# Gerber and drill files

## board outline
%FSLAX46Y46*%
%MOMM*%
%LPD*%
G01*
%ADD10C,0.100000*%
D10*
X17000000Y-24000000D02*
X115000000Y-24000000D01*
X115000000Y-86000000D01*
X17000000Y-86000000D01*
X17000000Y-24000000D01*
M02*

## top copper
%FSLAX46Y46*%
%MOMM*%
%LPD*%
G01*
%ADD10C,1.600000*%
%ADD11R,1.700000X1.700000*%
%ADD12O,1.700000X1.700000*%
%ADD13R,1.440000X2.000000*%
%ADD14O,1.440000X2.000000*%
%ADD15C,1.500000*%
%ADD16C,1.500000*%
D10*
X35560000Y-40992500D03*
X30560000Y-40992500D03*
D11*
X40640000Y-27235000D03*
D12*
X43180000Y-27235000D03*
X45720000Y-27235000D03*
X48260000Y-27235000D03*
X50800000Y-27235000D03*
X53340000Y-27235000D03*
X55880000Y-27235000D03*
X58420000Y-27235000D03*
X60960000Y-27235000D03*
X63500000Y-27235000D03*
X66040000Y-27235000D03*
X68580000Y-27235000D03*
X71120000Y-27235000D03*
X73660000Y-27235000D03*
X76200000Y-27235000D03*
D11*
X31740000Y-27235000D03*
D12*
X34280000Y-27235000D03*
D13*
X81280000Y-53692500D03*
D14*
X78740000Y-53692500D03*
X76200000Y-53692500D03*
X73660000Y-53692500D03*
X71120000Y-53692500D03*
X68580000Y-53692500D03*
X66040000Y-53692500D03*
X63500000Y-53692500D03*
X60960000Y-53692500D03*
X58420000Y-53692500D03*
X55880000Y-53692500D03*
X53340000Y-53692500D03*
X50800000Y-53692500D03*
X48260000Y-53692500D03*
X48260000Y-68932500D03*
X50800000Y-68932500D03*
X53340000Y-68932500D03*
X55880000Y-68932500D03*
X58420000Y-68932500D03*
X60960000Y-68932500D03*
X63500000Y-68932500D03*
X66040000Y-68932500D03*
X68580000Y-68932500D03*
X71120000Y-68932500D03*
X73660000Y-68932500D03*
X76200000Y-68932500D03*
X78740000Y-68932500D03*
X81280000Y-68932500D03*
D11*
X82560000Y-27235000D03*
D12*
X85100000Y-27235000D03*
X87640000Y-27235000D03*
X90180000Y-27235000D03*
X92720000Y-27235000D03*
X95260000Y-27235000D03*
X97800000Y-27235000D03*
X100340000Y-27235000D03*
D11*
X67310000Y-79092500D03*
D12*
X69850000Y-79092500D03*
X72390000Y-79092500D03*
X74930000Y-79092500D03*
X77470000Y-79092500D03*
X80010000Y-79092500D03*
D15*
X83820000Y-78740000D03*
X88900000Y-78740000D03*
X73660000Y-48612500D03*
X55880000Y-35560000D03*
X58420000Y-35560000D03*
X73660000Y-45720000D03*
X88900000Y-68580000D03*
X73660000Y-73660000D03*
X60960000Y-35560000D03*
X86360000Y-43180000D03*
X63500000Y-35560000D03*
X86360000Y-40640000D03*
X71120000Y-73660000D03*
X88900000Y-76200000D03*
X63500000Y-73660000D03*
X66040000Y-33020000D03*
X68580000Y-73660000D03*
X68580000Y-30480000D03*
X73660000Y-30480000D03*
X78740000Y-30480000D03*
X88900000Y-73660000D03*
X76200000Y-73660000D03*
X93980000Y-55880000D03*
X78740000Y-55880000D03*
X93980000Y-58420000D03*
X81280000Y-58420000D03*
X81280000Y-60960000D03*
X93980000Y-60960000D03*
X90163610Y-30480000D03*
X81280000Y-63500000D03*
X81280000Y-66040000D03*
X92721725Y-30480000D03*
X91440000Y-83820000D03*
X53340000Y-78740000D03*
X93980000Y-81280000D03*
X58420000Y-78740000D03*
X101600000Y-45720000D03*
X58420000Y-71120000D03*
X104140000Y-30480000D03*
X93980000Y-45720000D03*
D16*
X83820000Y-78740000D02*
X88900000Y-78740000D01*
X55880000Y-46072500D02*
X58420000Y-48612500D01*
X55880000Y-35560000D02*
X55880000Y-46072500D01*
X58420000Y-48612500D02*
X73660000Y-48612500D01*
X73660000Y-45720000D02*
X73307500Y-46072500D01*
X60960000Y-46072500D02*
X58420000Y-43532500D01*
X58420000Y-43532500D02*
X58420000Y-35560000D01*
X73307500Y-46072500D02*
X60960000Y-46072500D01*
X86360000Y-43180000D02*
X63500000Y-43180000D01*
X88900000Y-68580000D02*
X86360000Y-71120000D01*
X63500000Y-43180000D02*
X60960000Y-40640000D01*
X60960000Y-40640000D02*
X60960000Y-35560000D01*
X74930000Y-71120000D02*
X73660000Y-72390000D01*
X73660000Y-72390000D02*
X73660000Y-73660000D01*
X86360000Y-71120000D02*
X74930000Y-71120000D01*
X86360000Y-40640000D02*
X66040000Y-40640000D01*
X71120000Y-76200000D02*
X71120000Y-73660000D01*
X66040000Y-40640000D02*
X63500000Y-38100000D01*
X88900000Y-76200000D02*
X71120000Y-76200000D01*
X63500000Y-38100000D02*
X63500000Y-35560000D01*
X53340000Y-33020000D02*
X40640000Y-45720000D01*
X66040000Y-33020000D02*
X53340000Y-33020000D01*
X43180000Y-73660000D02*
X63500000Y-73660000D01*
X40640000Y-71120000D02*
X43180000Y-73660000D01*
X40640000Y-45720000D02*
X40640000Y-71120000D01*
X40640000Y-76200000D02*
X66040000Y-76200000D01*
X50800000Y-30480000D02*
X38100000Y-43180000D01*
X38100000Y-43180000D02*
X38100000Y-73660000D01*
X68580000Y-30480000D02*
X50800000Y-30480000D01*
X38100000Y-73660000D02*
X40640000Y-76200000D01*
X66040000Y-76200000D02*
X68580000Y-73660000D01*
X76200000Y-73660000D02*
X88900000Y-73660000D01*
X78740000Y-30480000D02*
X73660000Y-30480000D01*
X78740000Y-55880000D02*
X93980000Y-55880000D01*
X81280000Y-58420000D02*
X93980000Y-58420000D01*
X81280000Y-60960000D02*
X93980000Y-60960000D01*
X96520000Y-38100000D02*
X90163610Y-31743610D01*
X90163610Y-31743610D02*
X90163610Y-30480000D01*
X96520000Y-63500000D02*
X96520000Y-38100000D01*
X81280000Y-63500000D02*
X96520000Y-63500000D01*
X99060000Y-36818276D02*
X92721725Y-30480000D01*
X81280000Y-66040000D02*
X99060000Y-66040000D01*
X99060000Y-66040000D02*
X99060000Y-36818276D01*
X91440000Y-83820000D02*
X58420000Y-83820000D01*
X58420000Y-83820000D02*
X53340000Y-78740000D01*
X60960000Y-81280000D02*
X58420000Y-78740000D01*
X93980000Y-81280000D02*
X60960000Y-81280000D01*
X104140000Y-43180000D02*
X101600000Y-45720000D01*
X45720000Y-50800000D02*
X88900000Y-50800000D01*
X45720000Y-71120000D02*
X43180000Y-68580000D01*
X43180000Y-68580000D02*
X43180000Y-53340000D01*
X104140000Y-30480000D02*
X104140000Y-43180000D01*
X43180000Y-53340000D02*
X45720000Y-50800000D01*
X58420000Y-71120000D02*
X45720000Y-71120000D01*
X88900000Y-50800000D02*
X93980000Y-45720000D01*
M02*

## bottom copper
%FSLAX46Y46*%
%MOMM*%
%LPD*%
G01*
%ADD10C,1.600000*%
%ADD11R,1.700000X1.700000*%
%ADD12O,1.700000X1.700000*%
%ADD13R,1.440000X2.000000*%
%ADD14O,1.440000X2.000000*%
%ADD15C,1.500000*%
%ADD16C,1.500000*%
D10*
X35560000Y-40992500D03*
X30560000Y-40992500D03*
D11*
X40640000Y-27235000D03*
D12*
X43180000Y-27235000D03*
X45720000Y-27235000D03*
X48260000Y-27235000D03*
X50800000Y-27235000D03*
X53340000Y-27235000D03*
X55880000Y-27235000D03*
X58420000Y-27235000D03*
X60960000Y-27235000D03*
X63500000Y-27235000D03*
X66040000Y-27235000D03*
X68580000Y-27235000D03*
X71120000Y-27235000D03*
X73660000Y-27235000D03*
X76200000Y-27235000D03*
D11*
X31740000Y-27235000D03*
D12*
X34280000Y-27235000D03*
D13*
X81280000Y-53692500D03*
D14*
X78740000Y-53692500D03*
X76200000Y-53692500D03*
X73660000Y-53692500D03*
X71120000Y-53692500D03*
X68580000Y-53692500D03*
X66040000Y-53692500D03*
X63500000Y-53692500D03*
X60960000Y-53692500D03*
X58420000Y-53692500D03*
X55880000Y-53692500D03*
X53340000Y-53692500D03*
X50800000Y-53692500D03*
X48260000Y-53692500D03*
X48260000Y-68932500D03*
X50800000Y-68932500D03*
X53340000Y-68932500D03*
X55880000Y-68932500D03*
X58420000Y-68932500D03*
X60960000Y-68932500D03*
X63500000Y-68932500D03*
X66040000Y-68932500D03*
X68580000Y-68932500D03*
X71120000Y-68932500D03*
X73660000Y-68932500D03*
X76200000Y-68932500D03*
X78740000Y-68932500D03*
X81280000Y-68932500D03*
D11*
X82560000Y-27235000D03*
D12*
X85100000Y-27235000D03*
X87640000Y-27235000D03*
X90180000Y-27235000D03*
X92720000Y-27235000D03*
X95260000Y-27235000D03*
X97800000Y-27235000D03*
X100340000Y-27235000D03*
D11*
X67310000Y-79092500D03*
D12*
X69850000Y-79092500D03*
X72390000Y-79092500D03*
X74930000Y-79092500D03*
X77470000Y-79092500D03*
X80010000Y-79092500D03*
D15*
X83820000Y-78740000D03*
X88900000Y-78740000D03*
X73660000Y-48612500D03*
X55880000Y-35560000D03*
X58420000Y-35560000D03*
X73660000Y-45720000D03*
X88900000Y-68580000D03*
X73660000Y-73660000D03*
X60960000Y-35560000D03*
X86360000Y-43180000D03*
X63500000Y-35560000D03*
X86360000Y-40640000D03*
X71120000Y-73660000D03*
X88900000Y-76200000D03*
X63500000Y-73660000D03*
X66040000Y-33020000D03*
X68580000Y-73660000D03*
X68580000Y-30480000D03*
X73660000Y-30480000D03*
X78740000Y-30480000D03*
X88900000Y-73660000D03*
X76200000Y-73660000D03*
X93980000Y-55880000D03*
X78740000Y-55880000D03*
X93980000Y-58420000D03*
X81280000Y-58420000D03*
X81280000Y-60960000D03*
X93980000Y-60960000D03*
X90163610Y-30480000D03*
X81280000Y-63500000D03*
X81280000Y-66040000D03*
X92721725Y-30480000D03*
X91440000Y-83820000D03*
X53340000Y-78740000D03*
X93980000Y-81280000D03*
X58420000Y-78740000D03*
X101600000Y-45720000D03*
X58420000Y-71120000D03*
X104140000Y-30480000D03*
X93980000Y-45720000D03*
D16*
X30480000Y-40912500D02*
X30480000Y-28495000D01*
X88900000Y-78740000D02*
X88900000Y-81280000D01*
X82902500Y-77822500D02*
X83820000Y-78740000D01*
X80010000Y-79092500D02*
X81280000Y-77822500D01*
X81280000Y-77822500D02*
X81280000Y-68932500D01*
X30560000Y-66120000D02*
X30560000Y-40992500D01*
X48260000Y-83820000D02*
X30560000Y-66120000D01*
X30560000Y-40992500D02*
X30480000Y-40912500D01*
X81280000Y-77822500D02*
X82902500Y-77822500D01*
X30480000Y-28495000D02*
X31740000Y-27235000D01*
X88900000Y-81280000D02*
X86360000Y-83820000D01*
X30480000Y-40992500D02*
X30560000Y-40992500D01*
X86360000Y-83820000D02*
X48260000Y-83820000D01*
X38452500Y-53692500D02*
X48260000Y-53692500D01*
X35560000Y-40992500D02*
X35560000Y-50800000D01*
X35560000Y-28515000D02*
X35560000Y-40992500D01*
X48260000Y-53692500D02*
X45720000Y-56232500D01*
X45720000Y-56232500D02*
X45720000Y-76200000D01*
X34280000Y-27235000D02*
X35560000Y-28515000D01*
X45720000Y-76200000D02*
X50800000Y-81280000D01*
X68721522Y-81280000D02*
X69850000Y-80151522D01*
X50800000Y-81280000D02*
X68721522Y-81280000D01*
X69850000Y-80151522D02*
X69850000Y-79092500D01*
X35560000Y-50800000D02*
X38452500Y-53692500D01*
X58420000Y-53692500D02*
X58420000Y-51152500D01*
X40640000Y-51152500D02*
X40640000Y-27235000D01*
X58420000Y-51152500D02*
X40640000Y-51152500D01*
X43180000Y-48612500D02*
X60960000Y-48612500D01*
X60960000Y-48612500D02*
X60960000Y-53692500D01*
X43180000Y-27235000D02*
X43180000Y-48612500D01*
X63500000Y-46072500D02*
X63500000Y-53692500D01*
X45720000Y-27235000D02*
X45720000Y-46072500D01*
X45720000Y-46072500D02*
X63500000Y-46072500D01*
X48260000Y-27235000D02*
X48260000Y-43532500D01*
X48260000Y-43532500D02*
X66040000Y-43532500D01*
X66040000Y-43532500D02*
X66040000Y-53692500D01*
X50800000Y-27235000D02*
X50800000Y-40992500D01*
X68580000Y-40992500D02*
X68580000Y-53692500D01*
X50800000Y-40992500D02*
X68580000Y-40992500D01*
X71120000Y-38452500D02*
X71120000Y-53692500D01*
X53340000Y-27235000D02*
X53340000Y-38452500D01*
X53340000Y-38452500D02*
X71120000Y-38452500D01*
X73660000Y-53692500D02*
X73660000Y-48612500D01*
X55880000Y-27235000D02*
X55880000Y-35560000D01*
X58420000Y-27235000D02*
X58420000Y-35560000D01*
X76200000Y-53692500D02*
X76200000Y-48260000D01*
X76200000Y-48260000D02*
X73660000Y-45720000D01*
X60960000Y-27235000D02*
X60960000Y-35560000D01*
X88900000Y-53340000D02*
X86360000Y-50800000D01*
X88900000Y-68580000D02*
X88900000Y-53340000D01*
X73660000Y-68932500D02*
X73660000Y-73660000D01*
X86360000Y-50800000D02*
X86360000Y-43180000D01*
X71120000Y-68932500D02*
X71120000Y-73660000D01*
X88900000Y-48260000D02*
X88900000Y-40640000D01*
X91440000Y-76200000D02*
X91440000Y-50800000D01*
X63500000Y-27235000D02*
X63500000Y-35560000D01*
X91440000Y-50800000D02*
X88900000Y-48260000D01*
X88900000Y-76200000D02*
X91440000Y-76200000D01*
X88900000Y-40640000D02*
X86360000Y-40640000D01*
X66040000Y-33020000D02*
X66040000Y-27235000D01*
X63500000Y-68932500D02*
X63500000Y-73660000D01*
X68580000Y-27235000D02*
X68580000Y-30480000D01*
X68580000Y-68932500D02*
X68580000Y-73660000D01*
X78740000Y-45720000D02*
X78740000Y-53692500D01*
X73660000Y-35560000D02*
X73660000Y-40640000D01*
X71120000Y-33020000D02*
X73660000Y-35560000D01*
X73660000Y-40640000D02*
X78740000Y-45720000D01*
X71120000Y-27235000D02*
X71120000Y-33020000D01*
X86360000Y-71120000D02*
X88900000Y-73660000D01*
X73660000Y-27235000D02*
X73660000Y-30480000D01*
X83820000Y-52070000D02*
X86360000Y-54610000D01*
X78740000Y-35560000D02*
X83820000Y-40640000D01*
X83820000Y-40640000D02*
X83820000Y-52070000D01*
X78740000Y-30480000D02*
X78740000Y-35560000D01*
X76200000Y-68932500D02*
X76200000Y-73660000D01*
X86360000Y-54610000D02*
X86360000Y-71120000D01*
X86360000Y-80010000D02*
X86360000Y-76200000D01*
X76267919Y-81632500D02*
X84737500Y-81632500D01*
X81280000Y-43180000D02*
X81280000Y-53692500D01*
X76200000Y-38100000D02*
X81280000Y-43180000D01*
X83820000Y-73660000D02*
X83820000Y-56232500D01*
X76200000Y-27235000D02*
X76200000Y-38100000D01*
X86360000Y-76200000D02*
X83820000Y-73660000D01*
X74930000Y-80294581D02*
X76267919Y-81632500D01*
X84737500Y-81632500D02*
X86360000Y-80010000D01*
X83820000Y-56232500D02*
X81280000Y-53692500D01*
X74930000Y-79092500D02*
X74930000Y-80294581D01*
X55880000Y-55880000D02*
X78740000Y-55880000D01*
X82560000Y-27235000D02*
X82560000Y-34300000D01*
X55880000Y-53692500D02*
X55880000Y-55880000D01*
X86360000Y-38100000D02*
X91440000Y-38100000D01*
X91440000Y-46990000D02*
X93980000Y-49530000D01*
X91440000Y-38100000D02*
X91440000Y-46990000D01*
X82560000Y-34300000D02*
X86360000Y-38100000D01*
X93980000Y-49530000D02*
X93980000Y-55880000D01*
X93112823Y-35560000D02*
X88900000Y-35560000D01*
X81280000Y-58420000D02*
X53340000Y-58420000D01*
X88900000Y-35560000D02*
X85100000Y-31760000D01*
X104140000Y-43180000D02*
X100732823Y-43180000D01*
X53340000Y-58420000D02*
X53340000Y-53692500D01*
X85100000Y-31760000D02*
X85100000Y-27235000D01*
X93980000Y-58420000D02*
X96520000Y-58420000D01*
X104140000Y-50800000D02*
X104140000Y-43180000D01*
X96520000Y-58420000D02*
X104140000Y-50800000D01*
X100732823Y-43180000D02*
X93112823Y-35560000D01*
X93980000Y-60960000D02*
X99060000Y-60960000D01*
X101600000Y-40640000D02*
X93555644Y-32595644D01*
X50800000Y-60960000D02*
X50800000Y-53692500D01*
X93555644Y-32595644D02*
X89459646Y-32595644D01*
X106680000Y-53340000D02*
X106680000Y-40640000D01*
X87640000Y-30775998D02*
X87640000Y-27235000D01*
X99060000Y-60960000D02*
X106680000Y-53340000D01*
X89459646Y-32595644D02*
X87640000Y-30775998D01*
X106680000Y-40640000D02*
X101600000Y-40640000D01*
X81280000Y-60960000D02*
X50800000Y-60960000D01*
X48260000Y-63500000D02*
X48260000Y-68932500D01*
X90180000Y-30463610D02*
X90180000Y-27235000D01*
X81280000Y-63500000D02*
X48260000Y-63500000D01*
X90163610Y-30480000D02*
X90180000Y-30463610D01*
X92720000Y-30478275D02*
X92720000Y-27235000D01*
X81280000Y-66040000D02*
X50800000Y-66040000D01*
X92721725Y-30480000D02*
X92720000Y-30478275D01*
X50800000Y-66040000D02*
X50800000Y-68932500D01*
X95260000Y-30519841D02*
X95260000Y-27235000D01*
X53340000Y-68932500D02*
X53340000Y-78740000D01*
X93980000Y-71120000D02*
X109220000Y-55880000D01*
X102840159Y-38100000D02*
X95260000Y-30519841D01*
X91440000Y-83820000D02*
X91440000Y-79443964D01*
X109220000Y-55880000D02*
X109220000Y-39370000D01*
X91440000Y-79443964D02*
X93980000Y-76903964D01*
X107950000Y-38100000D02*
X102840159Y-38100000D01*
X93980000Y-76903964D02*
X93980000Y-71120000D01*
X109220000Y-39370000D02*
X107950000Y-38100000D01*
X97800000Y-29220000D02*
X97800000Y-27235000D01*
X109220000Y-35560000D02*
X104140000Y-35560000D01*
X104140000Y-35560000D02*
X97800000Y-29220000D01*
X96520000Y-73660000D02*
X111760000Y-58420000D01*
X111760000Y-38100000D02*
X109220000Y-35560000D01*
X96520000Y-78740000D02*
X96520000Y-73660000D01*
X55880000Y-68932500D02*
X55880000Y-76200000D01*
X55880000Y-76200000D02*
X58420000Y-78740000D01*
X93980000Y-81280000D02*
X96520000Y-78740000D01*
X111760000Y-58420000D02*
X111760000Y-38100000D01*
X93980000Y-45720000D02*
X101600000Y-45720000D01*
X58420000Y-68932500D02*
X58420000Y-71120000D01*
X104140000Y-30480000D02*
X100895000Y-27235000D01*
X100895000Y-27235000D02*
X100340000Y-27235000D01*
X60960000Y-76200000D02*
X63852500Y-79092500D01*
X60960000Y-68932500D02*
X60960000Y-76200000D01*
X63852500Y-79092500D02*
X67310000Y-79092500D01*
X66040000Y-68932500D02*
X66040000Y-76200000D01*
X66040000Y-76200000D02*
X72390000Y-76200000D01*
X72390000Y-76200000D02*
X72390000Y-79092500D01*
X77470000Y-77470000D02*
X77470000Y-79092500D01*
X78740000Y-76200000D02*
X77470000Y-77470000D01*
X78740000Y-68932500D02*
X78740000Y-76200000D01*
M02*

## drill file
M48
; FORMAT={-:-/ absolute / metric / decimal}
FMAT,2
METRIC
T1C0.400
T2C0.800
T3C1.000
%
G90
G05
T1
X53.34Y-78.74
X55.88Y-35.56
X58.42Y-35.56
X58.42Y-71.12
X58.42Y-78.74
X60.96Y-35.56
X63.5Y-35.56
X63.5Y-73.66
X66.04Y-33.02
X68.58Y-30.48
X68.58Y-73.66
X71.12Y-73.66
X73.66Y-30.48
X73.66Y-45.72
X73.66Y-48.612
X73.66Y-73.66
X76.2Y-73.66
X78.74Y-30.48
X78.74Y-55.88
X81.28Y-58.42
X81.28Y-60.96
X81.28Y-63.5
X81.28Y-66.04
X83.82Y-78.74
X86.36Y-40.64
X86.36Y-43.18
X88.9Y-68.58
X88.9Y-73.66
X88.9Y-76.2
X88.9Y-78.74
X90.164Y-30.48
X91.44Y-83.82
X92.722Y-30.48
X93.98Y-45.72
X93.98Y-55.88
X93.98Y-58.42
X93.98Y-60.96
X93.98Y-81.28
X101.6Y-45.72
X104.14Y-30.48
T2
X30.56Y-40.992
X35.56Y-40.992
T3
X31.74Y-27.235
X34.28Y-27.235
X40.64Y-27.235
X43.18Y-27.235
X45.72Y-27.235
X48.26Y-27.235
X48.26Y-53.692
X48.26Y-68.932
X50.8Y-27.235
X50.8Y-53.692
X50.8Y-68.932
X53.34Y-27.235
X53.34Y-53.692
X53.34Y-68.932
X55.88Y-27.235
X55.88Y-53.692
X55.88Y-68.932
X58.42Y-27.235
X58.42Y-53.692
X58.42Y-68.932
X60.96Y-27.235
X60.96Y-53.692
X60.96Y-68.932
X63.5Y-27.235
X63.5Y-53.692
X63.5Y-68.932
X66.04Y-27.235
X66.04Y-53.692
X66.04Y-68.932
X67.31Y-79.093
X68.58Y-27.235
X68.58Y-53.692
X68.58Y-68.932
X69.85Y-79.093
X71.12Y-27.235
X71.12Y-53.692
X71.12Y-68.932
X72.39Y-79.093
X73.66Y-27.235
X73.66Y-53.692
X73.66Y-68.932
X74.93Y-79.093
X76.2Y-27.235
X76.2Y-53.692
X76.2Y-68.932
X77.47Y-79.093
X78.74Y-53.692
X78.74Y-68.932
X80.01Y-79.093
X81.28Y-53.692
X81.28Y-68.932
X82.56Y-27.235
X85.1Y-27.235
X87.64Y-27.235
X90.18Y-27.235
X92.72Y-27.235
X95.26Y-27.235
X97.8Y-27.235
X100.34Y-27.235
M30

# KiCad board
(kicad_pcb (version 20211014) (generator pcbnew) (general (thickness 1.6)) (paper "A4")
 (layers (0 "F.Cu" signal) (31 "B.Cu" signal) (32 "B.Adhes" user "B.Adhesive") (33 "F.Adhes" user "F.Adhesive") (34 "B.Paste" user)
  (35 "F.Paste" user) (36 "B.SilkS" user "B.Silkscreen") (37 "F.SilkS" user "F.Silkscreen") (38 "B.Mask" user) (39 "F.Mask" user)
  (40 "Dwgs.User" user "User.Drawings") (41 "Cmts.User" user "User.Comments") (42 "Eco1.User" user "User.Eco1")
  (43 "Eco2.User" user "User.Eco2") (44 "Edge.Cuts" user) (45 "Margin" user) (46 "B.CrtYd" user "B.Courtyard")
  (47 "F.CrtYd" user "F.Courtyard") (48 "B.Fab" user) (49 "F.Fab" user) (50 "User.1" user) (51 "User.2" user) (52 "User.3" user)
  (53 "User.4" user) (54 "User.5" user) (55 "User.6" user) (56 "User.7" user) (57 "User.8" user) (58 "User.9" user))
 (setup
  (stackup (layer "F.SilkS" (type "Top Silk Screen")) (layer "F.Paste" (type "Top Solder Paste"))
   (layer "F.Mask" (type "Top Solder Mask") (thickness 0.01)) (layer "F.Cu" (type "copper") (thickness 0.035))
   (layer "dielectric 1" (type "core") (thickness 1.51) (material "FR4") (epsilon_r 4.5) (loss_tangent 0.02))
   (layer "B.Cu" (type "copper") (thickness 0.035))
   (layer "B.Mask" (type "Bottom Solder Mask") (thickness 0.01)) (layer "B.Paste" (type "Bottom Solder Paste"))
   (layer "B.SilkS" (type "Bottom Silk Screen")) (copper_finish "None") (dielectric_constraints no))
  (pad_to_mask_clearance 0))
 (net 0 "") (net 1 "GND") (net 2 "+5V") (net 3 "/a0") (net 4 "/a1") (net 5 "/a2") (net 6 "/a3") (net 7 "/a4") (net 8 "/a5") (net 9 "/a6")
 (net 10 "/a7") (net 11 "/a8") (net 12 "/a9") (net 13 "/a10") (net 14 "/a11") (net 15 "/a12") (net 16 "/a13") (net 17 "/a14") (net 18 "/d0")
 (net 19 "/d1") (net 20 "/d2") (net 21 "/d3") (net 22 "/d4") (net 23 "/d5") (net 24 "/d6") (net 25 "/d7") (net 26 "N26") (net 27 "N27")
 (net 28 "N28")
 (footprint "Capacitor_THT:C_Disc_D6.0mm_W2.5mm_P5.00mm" (layer "F.Cu") (at 35.56 40.9925 180)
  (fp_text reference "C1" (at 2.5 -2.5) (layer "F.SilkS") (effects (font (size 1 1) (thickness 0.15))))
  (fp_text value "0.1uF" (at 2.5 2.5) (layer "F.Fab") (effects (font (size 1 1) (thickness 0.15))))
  (pad "1" thru_hole circle locked (at 0 0 180) (size 1.6 1.6) (drill 0.8) (layers *.Cu *.Mask) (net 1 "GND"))
  (pad "2" thru_hole circle locked (at 5 0 180) (size 1.6 1.6) (drill 0.8) (layers *.Cu *.Mask) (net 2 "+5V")))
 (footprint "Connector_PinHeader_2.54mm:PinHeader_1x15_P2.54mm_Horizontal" (layer "F.Cu") (at 40.64 27.235 90)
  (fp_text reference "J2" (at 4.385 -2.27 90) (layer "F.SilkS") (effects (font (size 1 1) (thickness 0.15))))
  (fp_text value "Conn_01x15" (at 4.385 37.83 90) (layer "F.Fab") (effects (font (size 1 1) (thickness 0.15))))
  (pad "1" thru_hole rect locked (at 0 0 90) (size 1.7 1.7) (drill 1) (layers *.Cu *.Mask) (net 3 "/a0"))
  (pad "2" thru_hole oval locked (at 0 2.54 90) (size 1.7 1.7) (drill 1) (layers *.Cu *.Mask) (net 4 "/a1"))
  (pad "3" thru_hole oval locked (at 0 5.08 90) (size 1.7 1.7) (drill 1) (layers *.Cu *.Mask) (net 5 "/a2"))
  (pad "4" thru_hole oval locked (at 0 7.62 90) (size 1.7 1.7) (drill 1) (layers *.Cu *.Mask) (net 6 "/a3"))
  (pad "5" thru_hole oval locked (at 0 10.16 90) (size 1.7 1.7) (drill 1) (layers *.Cu *.Mask) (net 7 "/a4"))
  (pad "6" thru_hole oval locked (at 0 12.7 90) (size 1.7 1.7) (drill 1) (layers *.Cu *.Mask) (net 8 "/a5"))
  (pad "7" thru_hole oval locked (at 0 15.24 90) (size 1.7 1.7) (drill 1) (layers *.Cu *.Mask) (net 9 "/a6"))
  (pad "8" thru_hole oval locked (at 0 17.78 90) (size 1.7 1.7) (drill 1) (layers *.Cu *.Mask) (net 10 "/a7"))
  (pad "9" thru_hole oval locked (at 0 20.32 90) (size 1.7 1.7) (drill 1) (layers *.Cu *.Mask) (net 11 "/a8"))
  (pad "10" thru_hole oval locked (at 0 22.86 90) (size 1.7 1.7) (drill 1) (layers *.Cu *.Mask) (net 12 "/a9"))
  (pad "11" thru_hole oval locked (at 0 25.4 90) (size 1.7 1.7) (drill 1) (layers *.Cu *.Mask) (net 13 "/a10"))
  (pad "12" thru_hole oval locked (at 0 27.94 90) (size 1.7 1.7) (drill 1) (layers *.Cu *.Mask) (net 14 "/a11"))
  (pad "13" thru_hole oval locked (at 0 30.48 90) (size 1.7 1.7) (drill 1) (layers *.Cu *.Mask) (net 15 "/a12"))
  (pad "14" thru_hole oval locked (at 0 33.02 90) (size 1.7 1.7) (drill 1) (layers *.Cu *.Mask) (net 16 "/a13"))
  (pad "15" thru_hole oval locked (at 0 35.56 90) (size 1.7 1.7) (drill 1) (layers *.Cu *.Mask) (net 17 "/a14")))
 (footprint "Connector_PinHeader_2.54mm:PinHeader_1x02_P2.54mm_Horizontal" (layer "F.Cu") (at 31.74 27.235 90)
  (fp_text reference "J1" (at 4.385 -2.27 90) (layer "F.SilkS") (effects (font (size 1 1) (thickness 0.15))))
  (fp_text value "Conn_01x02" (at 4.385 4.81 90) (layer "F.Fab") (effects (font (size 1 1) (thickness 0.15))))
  (pad "1" thru_hole rect locked (at 0 0 90) (size 1.7 1.7) (drill 1) (layers *.Cu *.Mask) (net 2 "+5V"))
  (pad "2" thru_hole oval locked (at 0 2.54 90) (size 1.7 1.7) (drill 1) (layers *.Cu *.Mask) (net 1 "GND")))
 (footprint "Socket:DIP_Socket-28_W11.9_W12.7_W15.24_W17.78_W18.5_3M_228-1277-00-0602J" (layer "F.Cu") (at 81.28 53.6925 -90)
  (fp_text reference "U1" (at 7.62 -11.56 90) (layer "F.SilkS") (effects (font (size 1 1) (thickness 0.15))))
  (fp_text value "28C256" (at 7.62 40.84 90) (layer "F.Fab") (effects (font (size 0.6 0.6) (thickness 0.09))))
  (pad "1" thru_hole rect locked (at 0 0 270) (size 2 1.44) (drill 1) (layers *.Cu *.Mask) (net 17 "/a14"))
  (pad "2" thru_hole oval locked (at 0 2.54 270) (size 2 1.44) (drill 1) (layers *.Cu *.Mask) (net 15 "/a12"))
  (pad "3" thru_hole oval locked (at 0 5.08 270) (size 2 1.44) (drill 1) (layers *.Cu *.Mask) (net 10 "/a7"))
  (pad "4" thru_hole oval locked (at 0 7.62 270) (size 2 1.44) (drill 1) (layers *.Cu *.Mask) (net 9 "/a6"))
  (pad "5" thru_hole oval locked (at 0 10.16 270) (size 2 1.44) (drill 1) (layers *.Cu *.Mask) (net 8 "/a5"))
  (pad "6" thru_hole oval locked (at 0 12.7 270) (size 2 1.44) (drill 1) (layers *.Cu *.Mask) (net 7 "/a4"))
  (pad "7" thru_hole oval locked (at 0 15.24 270) (size 2 1.44) (drill 1) (layers *.Cu *.Mask) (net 6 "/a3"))
  (pad "8" thru_hole oval locked (at 0 17.78 270) (size 2 1.44) (drill 1) (layers *.Cu *.Mask) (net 5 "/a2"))
  (pad "9" thru_hole oval locked (at 0 20.32 270) (size 2 1.44) (drill 1) (layers *.Cu *.Mask) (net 4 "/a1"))
  (pad "10" thru_hole oval locked (at 0 22.86 270) (size 2 1.44) (drill 1) (layers *.Cu *.Mask) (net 3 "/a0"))
  (pad "11" thru_hole oval locked (at 0 25.4 270) (size 2 1.44) (drill 1) (layers *.Cu *.Mask) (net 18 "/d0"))
  (pad "12" thru_hole oval locked (at 0 27.94 270) (size 2 1.44) (drill 1) (layers *.Cu *.Mask) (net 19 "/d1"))
  (pad "13" thru_hole oval locked (at 0 30.48 270) (size 2 1.44) (drill 1) (layers *.Cu *.Mask) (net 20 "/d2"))
  (pad "14" thru_hole oval locked (at 0 33.02 270) (size 2 1.44) (drill 1) (layers *.Cu *.Mask) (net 1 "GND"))
  (pad "15" thru_hole oval locked (at 15.24 33.02 270) (size 2 1.44) (drill 1) (layers *.Cu *.Mask) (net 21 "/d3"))
  (pad "16" thru_hole oval locked (at 15.24 30.48 270) (size 2 1.44) (drill 1) (layers *.Cu *.Mask) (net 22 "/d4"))
  (pad "17" thru_hole oval locked (at 15.24 27.94 270) (size 2 1.44) (drill 1) (layers *.Cu *.Mask) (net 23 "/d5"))
  (pad "18" thru_hole oval locked (at 15.24 25.4 270) (size 2 1.44) (drill 1) (layers *.Cu *.Mask) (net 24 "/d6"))
  (pad "19" thru_hole oval locked (at 15.24 22.86 270) (size 2 1.44) (drill 1) (layers *.Cu *.Mask) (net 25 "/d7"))
  (pad "20" thru_hole oval locked (at 15.24 20.32 270) (size 2 1.44) (drill 1) (layers *.Cu *.Mask) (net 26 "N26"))
  (pad "21" thru_hole oval locked (at 15.24 17.78 270) (size 2 1.44) (drill 1) (layers *.Cu *.Mask) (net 13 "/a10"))
  (pad "22" thru_hole oval locked (at 15.24 15.24 270) (size 2 1.44) (drill 1) (layers *.Cu *.Mask) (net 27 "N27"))
  (pad "23" thru_hole oval locked (at 15.24 12.7 270) (size 2 1.44) (drill 1) (layers *.Cu *.Mask) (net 14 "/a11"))
  (pad "24" thru_hole oval locked (at 15.24 10.16 270) (size 2 1.44) (drill 1) (layers *.Cu *.Mask) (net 12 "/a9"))
  (pad "25" thru_hole oval locked (at 15.24 7.62 270) (size 2 1.44) (drill 1) (layers *.Cu *.Mask) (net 11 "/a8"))
  (pad "26" thru_hole oval locked (at 15.24 5.08 270) (size 2 1.44) (drill 1) (layers *.Cu *.Mask) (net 16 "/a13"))
  (pad "27" thru_hole oval locked (at 15.24 2.54 270) (size 2 1.44) (drill 1) (layers *.Cu *.Mask) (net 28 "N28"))
  (pad "28" thru_hole oval locked (at 15.24 0 270) (size 2 1.44) (drill 1) (layers *.Cu *.Mask) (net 2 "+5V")))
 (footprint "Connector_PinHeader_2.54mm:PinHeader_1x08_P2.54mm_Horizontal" (layer "F.Cu") (at 82.56 27.235 90)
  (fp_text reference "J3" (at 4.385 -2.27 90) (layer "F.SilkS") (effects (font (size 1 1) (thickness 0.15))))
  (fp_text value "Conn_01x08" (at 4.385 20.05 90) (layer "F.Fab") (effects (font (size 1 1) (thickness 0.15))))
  (pad "1" thru_hole rect locked (at 0 0 90) (size 1.7 1.7) (drill 1) (layers *.Cu *.Mask) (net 18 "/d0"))
  (pad "2" thru_hole oval locked (at 0 2.54 90) (size 1.7 1.7) (drill 1) (layers *.Cu *.Mask) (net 19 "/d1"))
  (pad "3" thru_hole oval locked (at 0 5.08 90) (size 1.7 1.7) (drill 1) (layers *.Cu *.Mask) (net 20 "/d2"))
  (pad "4" thru_hole oval locked (at 0 7.62 90) (size 1.7 1.7) (drill 1) (layers *.Cu *.Mask) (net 21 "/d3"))
  (pad "5" thru_hole oval locked (at 0 10.16 90) (size 1.7 1.7) (drill 1) (layers *.Cu *.Mask) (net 22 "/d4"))
  (pad "6" thru_hole oval locked (at 0 12.7 90) (size 1.7 1.7) (drill 1) (layers *.Cu *.Mask) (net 23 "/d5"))
  (pad "7" thru_hole oval locked (at 0 15.24 90) (size 1.7 1.7) (drill 1) (layers *.Cu *.Mask) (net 24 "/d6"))
  (pad "8" thru_hole oval locked (at 0 17.78 90) (size 1.7 1.7) (drill 1) (layers *.Cu *.Mask) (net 25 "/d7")))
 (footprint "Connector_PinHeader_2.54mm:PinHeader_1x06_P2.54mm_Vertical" (layer "F.Cu") (at 67.31 79.0925 90)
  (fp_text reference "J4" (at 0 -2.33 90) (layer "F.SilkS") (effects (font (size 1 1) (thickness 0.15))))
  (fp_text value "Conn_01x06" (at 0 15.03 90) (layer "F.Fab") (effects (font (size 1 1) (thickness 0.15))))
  (pad "1" thru_hole rect locked (at 0 0 90) (size 1.7 1.7) (drill 1) (layers *.Cu *.Mask) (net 26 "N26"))
  (pad "2" thru_hole oval locked (at 0 2.54 90) (size 1.7 1.7) (drill 1) (layers *.Cu *.Mask) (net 1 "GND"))
  (pad "3" thru_hole oval locked (at 0 5.08 90) (size 1.7 1.7) (drill 1) (layers *.Cu *.Mask) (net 27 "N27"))
  (pad "4" thru_hole oval locked (at 0 7.62 90) (size 1.7 1.7) (drill 1) (layers *.Cu *.Mask) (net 17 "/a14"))
  (pad "5" thru_hole oval locked (at 0 10.16 90) (size 1.7 1.7) (drill 1) (layers *.Cu *.Mask) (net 28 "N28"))
  (pad "6" thru_hole oval locked (at 0 12.7 90) (size 1.7 1.7) (drill 1) (layers *.Cu *.Mask) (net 2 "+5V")))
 (gr_rect (start 17 24) (end 115 86) (layer "Edge.Cuts") (width 0.1) (fill none))
 (segment (start 83.82 78.74) (end 88.9 78.74) (width 1.5) (layer "F.Cu") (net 2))
 (via (at 83.82 78.74) (size 1.5) (drill 0.4) (layers "F.Cu" "B.Cu") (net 2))
 (via (at 88.9 78.74) (size 1.5) (drill 0.4) (layers "F.Cu" "B.Cu") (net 2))
 (segment (start 30.48 40.9125) (end 30.48 28.495) (width 1.5) (layer "B.Cu") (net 2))
 (segment (start 88.9 78.74) (end 88.9 81.28) (width 1.5) (layer "B.Cu") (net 2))
 (segment (start 82.9025 77.8225) (end 83.82 78.74) (width 1.5) (layer "B.Cu") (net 2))
 (segment (start 80.01 79.0925) (end 81.28 77.8225) (width 1.5) (layer "B.Cu") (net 2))
 (segment (start 81.28 77.8225) (end 81.28 68.9325) (width 1.5) (layer "B.Cu") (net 2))
 (segment (start 30.56 66.12) (end 30.56 40.9925) (width 1.5) (layer "B.Cu") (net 2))
 (segment (start 48.26 83.82) (end 30.56 66.12) (width 1.5) (layer "B.Cu") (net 2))
 (segment (start 30.56 40.9925) (end 30.48 40.9125) (width 1.5) (layer "B.Cu") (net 2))
 (segment (start 81.28 77.8225) (end 82.9025 77.8225) (width 1.5) (layer "B.Cu") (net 2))
 (segment (start 30.48 28.495) (end 31.74 27.235) (width 1.5) (layer "B.Cu") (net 2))
 (segment (start 88.9 81.28) (end 86.36 83.82) (width 1.5) (layer "B.Cu") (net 2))
 (segment (start 30.48 40.9925) (end 30.56 40.9925) (width 1.5) (layer "B.Cu") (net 2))
 (segment (start 86.36 83.82) (end 48.26 83.82) (width 1.5) (layer "B.Cu") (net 2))
 (segment (start 38.4525 53.6925) (end 48.26 53.6925) (width 1.5) (layer "B.Cu") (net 1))
 (segment (start 35.56 40.9925) (end 35.56 50.8) (width 1.5) (layer "B.Cu") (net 1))
 (segment (start 35.56 28.515) (end 35.56 40.9925) (width 1.5) (layer "B.Cu") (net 1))
 (segment (start 48.26 53.6925) (end 45.72 56.2325) (width 1.5) (layer "B.Cu") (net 1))
 (segment (start 45.72 56.2325) (end 45.72 76.2) (width 1.5) (layer "B.Cu") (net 1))
 (segment (start 34.28 27.235) (end 35.56 28.515) (width 1.5) (layer "B.Cu") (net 1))
 (segment (start 45.72 76.2) (end 50.8 81.28) (width 1.5) (layer "B.Cu") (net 1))
 (segment (start 68.721522 81.28) (end 69.85 80.151522) (width 1.5) (layer "B.Cu") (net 1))
 (segment (start 50.8 81.28) (end 68.721522 81.28) (width 1.5) (layer "B.Cu") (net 1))
 (segment (start 69.85 80.151522) (end 69.85 79.0925) (width 1.5) (layer "B.Cu") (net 1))
 (segment (start 35.56 50.8) (end 38.4525 53.6925) (width 1.5) (layer "B.Cu") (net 1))
 (segment (start 58.42 53.6925) (end 58.42 51.1525) (width 1.5) (layer "B.Cu") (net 3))
 (segment (start 40.64 51.1525) (end 40.64 27.235) (width 1.5) (layer "B.Cu") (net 3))
 (segment (start 58.42 51.1525) (end 40.64 51.1525) (width 1.5) (layer "B.Cu") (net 3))
 (segment (start 43.18 48.6125) (end 60.96 48.6125) (width 1.5) (layer "B.Cu") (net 4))
 (segment (start 60.96 48.6125) (end 60.96 53.6925) (width 1.5) (layer "B.Cu") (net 4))
 (segment (start 43.18 27.235) (end 43.18 48.6125) (width 1.5) (layer "B.Cu") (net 4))
 (segment (start 63.5 46.0725) (end 63.5 53.6925) (width 1.5) (layer "B.Cu") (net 5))
 (segment (start 45.72 27.235) (end 45.72 46.0725) (width 1.5) (layer "B.Cu") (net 5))
 (segment (start 45.72 46.0725) (end 63.5 46.0725) (width 1.5) (layer "B.Cu") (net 5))
 (segment (start 48.26 27.235) (end 48.26 43.5325) (width 1.5) (layer "B.Cu") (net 6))
 (segment (start 48.26 43.5325) (end 66.04 43.5325) (width 1.5) (layer "B.Cu") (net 6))
 (segment (start 66.04 43.5325) (end 66.04 53.6925) (width 1.5) (layer "B.Cu") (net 6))
 (segment (start 50.8 27.235) (end 50.8 40.9925) (width 1.5) (layer "B.Cu") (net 7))
 (segment (start 68.58 40.9925) (end 68.58 53.6925) (width 1.5) (layer "B.Cu") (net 7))
 (segment (start 50.8 40.9925) (end 68.58 40.9925) (width 1.5) (layer "B.Cu") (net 7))
 (segment (start 71.12 38.4525) (end 71.12 53.6925) (width 1.5) (layer "B.Cu") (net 8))
 (segment (start 53.34 27.235) (end 53.34 38.4525) (width 1.5) (layer "B.Cu") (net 8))
 (segment (start 53.34 38.4525) (end 71.12 38.4525) (width 1.5) (layer "B.Cu") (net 8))
 (segment (start 55.88 46.0725) (end 58.42 48.6125) (width 1.5) (layer "F.Cu") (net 9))
 (segment (start 55.88 35.56) (end 55.88 46.0725) (width 1.5) (layer "F.Cu") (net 9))
 (segment (start 58.42 48.6125) (end 73.66 48.6125) (width 1.5) (layer "F.Cu") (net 9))
 (via (at 73.66 48.6125) (size 1.5) (drill 0.4) (layers "F.Cu" "B.Cu") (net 9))
 (via (at 55.88 35.56) (size 1.5) (drill 0.4) (layers "F.Cu" "B.Cu") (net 9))
 (segment (start 73.66 53.6925) (end 73.66 48.6125) (width 1.5) (layer "B.Cu") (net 9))
 (segment (start 55.88 27.235) (end 55.88 35.56) (width 1.5) (layer "B.Cu") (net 9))
 (segment (start 73.66 45.72) (end 73.3075 46.0725) (width 1.5) (layer "F.Cu") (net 10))
 (segment (start 60.96 46.0725) (end 58.42 43.5325) (width 1.5) (layer "F.Cu") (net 10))
 (segment (start 58.42 43.5325) (end 58.42 35.56) (width 1.5) (layer "F.Cu") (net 10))
 (segment (start 73.3075 46.0725) (end 60.96 46.0725) (width 1.5) (layer "F.Cu") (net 10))
 (via (at 58.42 35.56) (size 1.5) (drill 0.4) (layers "F.Cu" "B.Cu") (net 10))
 (via (at 73.66 45.72) (size 1.5) (drill 0.4) (layers "F.Cu" "B.Cu") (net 10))
 (segment (start 58.42 27.235) (end 58.42 35.56) (width 1.5) (layer "B.Cu") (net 10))
 (segment (start 76.2 53.6925) (end 76.2 48.26) (width 1.5) (layer "B.Cu") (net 10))
 (segment (start 76.2 48.26) (end 73.66 45.72) (width 1.5) (layer "B.Cu") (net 10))
 (segment (start 86.36 43.18) (end 63.5 43.18) (width 1.5) (layer "F.Cu") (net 11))
 (segment (start 88.9 68.58) (end 86.36 71.12) (width 1.5) (layer "F.Cu") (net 11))
 (segment (start 63.5 43.18) (end 60.96 40.64) (width 1.5) (layer "F.Cu") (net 11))
 (segment (start 60.96 40.64) (end 60.96 35.56) (width 1.5) (layer "F.Cu") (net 11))
 (segment (start 74.93 71.12) (end 73.66 72.39) (width 1.5) (layer "F.Cu") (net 11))
 (segment (start 73.66 72.39) (end 73.66 73.66) (width 1.5) (layer "F.Cu") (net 11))
 (segment (start 86.36 71.12) (end 74.93 71.12) (width 1.5) (layer "F.Cu") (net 11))
 (via (at 88.9 68.58) (size 1.5) (drill 0.4) (layers "F.Cu" "B.Cu") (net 11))
 (via (at 73.66 73.66) (size 1.5) (drill 0.4) (layers "F.Cu" "B.Cu") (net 11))
 (via (at 60.96 35.56) (size 1.5) (drill 0.4) (layers "F.Cu" "B.Cu") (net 11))
 (via (at 86.36 43.18) (size 1.5) (drill 0.4) (layers "F.Cu" "B.Cu") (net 11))
 (segment (start 60.96 27.235) (end 60.96 35.56) (width 1.5) (layer "B.Cu") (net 11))
 (segment (start 88.9 53.34) (end 86.36 50.8) (width 1.5) (layer "B.Cu") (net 11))
 (segment (start 88.9 68.58) (end 88.9 53.34) (width 1.5) (layer "B.Cu") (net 11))
 (segment (start 73.66 68.9325) (end 73.66 73.66) (width 1.5) (layer "B.Cu") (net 11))
 (segment (start 86.36 50.8) (end 86.36 43.18) (width 1.5) (layer "B.Cu") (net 11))
 (segment (start 86.36 40.64) (end 66.04 40.64) (width 1.5) (layer "F.Cu") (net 12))
 (segment (start 71.12 76.2) (end 71.12 73.66) (width 1.5) (layer "F.Cu") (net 12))
 (segment (start 66.04 40.64) (end 63.5 38.1) (width 1.5) (layer "F.Cu") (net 12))
 (segment (start 88.9 76.2) (end 71.12 76.2) (width 1.5) (layer "F.Cu") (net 12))
 (segment (start 63.5 38.1) (end 63.5 35.56) (width 1.5) (layer "F.Cu") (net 12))
 (via (at 63.5 35.56) (size 1.5) (drill 0.4) (layers "F.Cu" "B.Cu") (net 12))
 (via (at 86.36 40.64) (size 1.5) (drill 0.4) (layers "F.Cu" "B.Cu") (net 12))
 (via (at 71.12 73.66) (size 1.5) (drill 0.4) (layers "F.Cu" "B.Cu") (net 12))
 (via (at 88.9 76.2) (size 1.5) (drill 0.4) (layers "F.Cu" "B.Cu") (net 12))
 (segment (start 71.12 68.9325) (end 71.12 73.66) (width 1.5) (layer "B.Cu") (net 12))
 (segment (start 88.9 48.26) (end 88.9 40.64) (width 1.5) (layer "B.Cu") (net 12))
 (segment (start 91.44 76.2) (end 91.44 50.8) (width 1.5) (layer "B.Cu") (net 12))
 (segment (start 63.5 27.235) (end 63.5 35.56) (width 1.5) (layer "B.Cu") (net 12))
 (segment (start 91.44 50.8) (end 88.9 48.26) (width 1.5) (layer "B.Cu") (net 12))
 (segment (start 88.9 76.2) (end 91.44 76.2) (width 1.5) (layer "B.Cu") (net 12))
 (segment (start 88.9 40.64) (end 86.36 40.64) (width 1.5) (layer "B.Cu") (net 12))
 (segment (start 53.34 33.02) (end 40.64 45.72) (width 1.5) (layer "F.Cu") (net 13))
 (segment (start 66.04 33.02) (end 53.34 33.02) (width 1.5) (layer "F.Cu") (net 13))
 (segment (start 43.18 73.66) (end 63.5 73.66) (width 1.5) (layer "F.Cu") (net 13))
 (segment (start 40.64 71.12) (end 43.18 73.66) (width 1.5) (layer "F.Cu") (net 13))
 (segment (start 40.64 45.72) (end 40.64 71.12) (width 1.5) (layer "F.Cu") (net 13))
 (via (at 63.5 73.66) (size 1.5) (drill 0.4) (layers "F.Cu" "B.Cu") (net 13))
 (via (at 66.04 33.02) (size 1.5) (drill 0.4) (layers "F.Cu" "B.Cu") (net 13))
 (segment (start 66.04 33.02) (end 66.04 27.235) (width 1.5) (layer "B.Cu") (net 13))
 (segment (start 63.5 68.9325) (end 63.5 73.66) (width 1.5) (layer "B.Cu") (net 13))
 (segment (start 40.64 76.2) (end 66.04 76.2) (width 1.5) (layer "F.Cu") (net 14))
 (segment (start 50.8 30.48) (end 38.1 43.18) (width 1.5) (layer "F.Cu") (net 14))
 (segment (start 38.1 43.18) (end 38.1 73.66) (width 1.5) (layer "F.Cu") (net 14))
 (segment (start 68.58 30.48) (end 50.8 30.48) (width 1.5) (layer "F.Cu") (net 14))
 (segment (start 38.1 73.66) (end 40.64 76.2) (width 1.5) (layer "F.Cu") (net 14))
 (segment (start 66.04 76.2) (end 68.58 73.66) (width 1.5) (layer "F.Cu") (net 14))
 (via (at 68.58 73.66) (size 1.5) (drill 0.4) (layers "F.Cu" "B.Cu") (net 14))
 (via (at 68.58 30.48) (size 1.5) (drill 0.4) (layers "F.Cu" "B.Cu") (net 14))
 (segment (start 68.58 27.235) (end 68.58 30.48) (width 1.5) (layer "B.Cu") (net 14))
 (segment (start 68.58 68.9325) (end 68.58 73.66) (width 1.5) (layer "B.Cu") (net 14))
 (segment (start 78.74 45.72) (end 78.74 53.6925) (width 1.5) (layer "B.Cu") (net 15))
 (segment (start 73.66 35.56) (end 73.66 40.64) (width 1.5) (layer "B.Cu") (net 15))
 (segment (start 71.12 33.02) (end 73.66 35.56) (width 1.5) (layer "B.Cu") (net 15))
 (segment (start 73.66 40.64) (end 78.74 45.72) (width 1.5) (layer "B.Cu") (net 15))
 (segment (start 71.12 27.235) (end 71.12 33.02) (width 1.5) (layer "B.Cu") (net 15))
 (segment (start 76.2 73.66) (end 88.9 73.66) (width 1.5) (layer "F.Cu") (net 16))
 (segment (start 78.74 30.48) (end 73.66 30.48) (width 1.5) (layer "F.Cu") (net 16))
 (via (at 73.66 30.48) (size 1.5) (drill 0.4) (layers "F.Cu" "B.Cu") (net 16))
 (via (at 78.74 30.48) (size 1.5) (drill 0.4) (layers "F.Cu" "B.Cu") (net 16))
 (via (at 88.9 73.66) (size 1.5) (drill 0.4) (layers "F.Cu" "B.Cu") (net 16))
 (via (at 76.2 73.66) (size 1.5) (drill 0.4) (layers "F.Cu" "B.Cu") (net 16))
 (segment (start 86.36 71.12) (end 88.9 73.66) (width 1.5) (layer "B.Cu") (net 16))
 (segment (start 73.66 27.235) (end 73.66 30.48) (width 1.5) (layer "B.Cu") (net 16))
 (segment (start 83.82 52.07) (end 86.36 54.61) (width 1.5) (layer "B.Cu") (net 16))
 (segment (start 78.74 35.56) (end 83.82 40.64) (width 1.5) (layer "B.Cu") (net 16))
 (segment (start 83.82 40.64) (end 83.82 52.07) (width 1.5) (layer "B.Cu") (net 16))
 (segment (start 78.74 30.48) (end 78.74 35.56) (width 1.5) (layer "B.Cu") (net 16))
 (segment (start 76.2 68.9325) (end 76.2 73.66) (width 1.5) (layer "B.Cu") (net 16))
 (segment (start 86.36 54.61) (end 86.36 71.12) (width 1.5) (layer "B.Cu") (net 16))
 (segment (start 86.36 80.01) (end 86.36 76.2) (width 1.5) (layer "B.Cu") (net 17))
 (segment (start 76.267919 81.6325) (end 84.7375 81.6325) (width 1.5) (layer "B.Cu") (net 17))
 (segment (start 81.28 43.18) (end 81.28 53.6925) (width 1.5) (layer "B.Cu") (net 17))
 (segment (start 76.2 38.1) (end 81.28 43.18) (width 1.5) (layer "B.Cu") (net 17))
 (segment (start 83.82 73.66) (end 83.82 56.2325) (width 1.5) (layer "B.Cu") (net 17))
 (segment (start 76.2 27.235) (end 76.2 38.1) (width 1.5) (layer "B.Cu") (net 17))
 (segment (start 86.36 76.2) (end 83.82 73.66) (width 1.5) (layer "B.Cu") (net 17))
 (segment (start 74.93 80.294581) (end 76.267919 81.6325) (width 1.5) (layer "B.Cu") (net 17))
 (segment (start 84.7375 81.6325) (end 86.36 80.01) (width 1.5) (layer "B.Cu") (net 17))
 (segment (start 83.82 56.2325) (end 81.28 53.6925) (width 1.5) (layer "B.Cu") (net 17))
 (segment (start 74.93 79.0925) (end 74.93 80.294581) (width 1.5) (layer "B.Cu") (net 17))
 (segment (start 78.74 55.88) (end 93.98 55.88) (width 1.5) (layer "F.Cu") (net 18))
 (via (at 93.98 55.88) (size 1.5) (drill 0.4) (layers "F.Cu" "B.Cu") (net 18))
 (via (at 78.74 55.88) (size 1.5) (drill 0.4) (layers "F.Cu" "B.Cu") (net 18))
 (segment (start 55.88 55.88) (end 78.74 55.88) (width 1.5) (layer "B.Cu") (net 18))
 (segment (start 82.56 27.235) (end 82.56 34.3) (width 1.5) (layer "B.Cu") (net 18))
 (segment (start 55.88 53.6925) (end 55.88 55.88) (width 1.5) (layer "B.Cu") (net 18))
 (segment (start 86.36 38.1) (end 91.44 38.1) (width 1.5) (layer "B.Cu") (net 18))
 (segment (start 91.44 46.99) (end 93.98 49.53) (width 1.5) (layer "B.Cu") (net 18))
 (segment (start 91.44 38.1) (end 91.44 46.99) (width 1.5) (layer "B.Cu") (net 18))
 (segment (start 82.56 34.3) (end 86.36 38.1) (width 1.5) (layer "B.Cu") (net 18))
 (segment (start 93.98 49.53) (end 93.98 55.88) (width 1.5) (layer "B.Cu") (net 18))
 (segment (start 81.28 58.42) (end 93.98 58.42) (width 1.5) (layer "F.Cu") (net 19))
 (via (at 93.98 58.42) (size 1.5) (drill 0.4) (layers "F.Cu" "B.Cu") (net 19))
 (via (at 81.28 58.42) (size 1.5) (drill 0.4) (layers "F.Cu" "B.Cu") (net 19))
 (segment (start 93.112823 35.56) (end 88.9 35.56) (width 1.5) (layer "B.Cu") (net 19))
 (segment (start 81.28 58.42) (end 53.34 58.42) (width 1.5) (layer "B.Cu") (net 19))
 (segment (start 88.9 35.56) (end 85.1 31.76) (width 1.5) (layer "B.Cu") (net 19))
 (segment (start 104.14 43.18) (end 100.732823 43.18) (width 1.5) (layer "B.Cu") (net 19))
 (segment (start 53.34 58.42) (end 53.34 53.6925) (width 1.5) (layer "B.Cu") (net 19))
 (segment (start 85.1 31.76) (end 85.1 27.235) (width 1.5) (layer "B.Cu") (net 19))
 (segment (start 93.98 58.42) (end 96.52 58.42) (width 1.5) (layer "B.Cu") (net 19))
 (segment (start 104.14 50.8) (end 104.14 43.18) (width 1.5) (layer "B.Cu") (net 19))
 (segment (start 96.52 58.42) (end 104.14 50.8) (width 1.5) (layer "B.Cu") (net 19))
 (segment (start 100.732823 43.18) (end 93.112823 35.56) (width 1.5) (layer "B.Cu") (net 19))
 (segment (start 81.28 60.96) (end 93.98 60.96) (width 1.5) (layer "F.Cu") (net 20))
 (via (at 81.28 60.96) (size 1.5) (drill 0.4) (layers "F.Cu" "B.Cu") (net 20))
 (via (at 93.98 60.96) (size 1.5) (drill 0.4) (layers "F.Cu" "B.Cu") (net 20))
 (segment (start 93.98 60.96) (end 99.06 60.96) (width 1.5) (layer "B.Cu") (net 20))
 (segment (start 101.6 40.64) (end 93.555644 32.595644) (width 1.5) (layer "B.Cu") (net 20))
 (segment (start 50.8 60.96) (end 50.8 53.6925) (width 1.5) (layer "B.Cu") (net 20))
 (segment (start 93.555644 32.595644) (end 89.459646 32.595644) (width 1.5) (layer "B.Cu") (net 20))
 (segment (start 106.68 53.34) (end 106.68 40.64) (width 1.5) (layer "B.Cu") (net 20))
 (segment (start 87.64 30.775998) (end 87.64 27.235) (width 1.5) (layer "B.Cu") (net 20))
 (segment (start 99.06 60.96) (end 106.68 53.34) (width 1.5) (layer "B.Cu") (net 20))
 (segment (start 89.459646 32.595644) (end 87.64 30.775998) (width 1.5) (layer "B.Cu") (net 20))
 (segment (start 106.68 40.64) (end 101.6 40.64) (width 1.5) (layer "B.Cu") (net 20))
 (segment (start 81.28 60.96) (end 50.8 60.96) (width 1.5) (layer "B.Cu") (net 20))
 (segment (start 96.52 38.1) (end 90.16361 31.74361) (width 1.5) (layer "F.Cu") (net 21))
 (segment (start 90.16361 31.74361) (end 90.16361 30.48) (width 1.5) (layer "F.Cu") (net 21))
 (segment (start 96.52 63.5) (end 96.52 38.1) (width 1.5) (layer "F.Cu") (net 21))
 (segment (start 81.28 63.5) (end 96.52 63.5) (width 1.5) (layer "F.Cu") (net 21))
 (via (at 90.16361 30.48) (size 1.5) (drill 0.4) (layers "F.Cu" "B.Cu") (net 21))
 (via (at 81.28 63.5) (size 1.5) (drill 0.4) (layers "F.Cu" "B.Cu") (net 21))
 (segment (start 48.26 63.5) (end 48.26 68.9325) (width 1.5) (layer "B.Cu") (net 21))
 (segment (start 90.18 30.46361) (end 90.18 27.235) (width 1.5) (layer "B.Cu") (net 21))
 (segment (start 81.28 63.5) (end 48.26 63.5) (width 1.5) (layer "B.Cu") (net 21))
 (segment (start 90.16361 30.48) (end 90.18 30.46361) (width 1.5) (layer "B.Cu") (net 21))
 (segment (start 99.06 36.818276) (end 92.721725 30.48) (width 1.5) (layer "F.Cu") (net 22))
 (segment (start 81.28 66.04) (end 99.06 66.04) (width 1.5) (layer "F.Cu") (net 22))
 (segment (start 99.06 66.04) (end 99.06 36.818276) (width 1.5) (layer "F.Cu") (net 22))
 (via (at 81.28 66.04) (size 1.5) (drill 0.4) (layers "F.Cu" "B.Cu") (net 22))
 (via (at 92.721725 30.48) (size 1.5) (drill 0.4) (layers "F.Cu" "B.Cu") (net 22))
 (segment (start 92.72 30.478275) (end 92.72 27.235) (width 1.5) (layer "B.Cu") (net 22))
 (segment (start 81.28 66.04) (end 50.8 66.04) (width 1.5) (layer "B.Cu") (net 22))
 (segment (start 92.721725 30.48) (end 92.72 30.478275) (width 1.5) (layer "B.Cu") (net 22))
 (segment (start 50.8 66.04) (end 50.8 68.9325) (width 1.5) (layer "B.Cu") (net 22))
 (segment (start 91.44 83.82) (end 58.42 83.82) (width 1.5) (layer "F.Cu") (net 23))
 (segment (start 58.42 83.82) (end 53.34 78.74) (width 1.5) (layer "F.Cu") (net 23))
 (via (at 91.44 83.82) (size 1.5) (drill 0.4) (layers "F.Cu" "B.Cu") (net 23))
 (via (at 53.34 78.74) (size 1.5) (drill 0.4) (layers "F.Cu" "B.Cu") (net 23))
 (segment (start 95.26 30.519841) (end 95.26 27.235) (width 1.5) (layer "B.Cu") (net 23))
 (segment (start 53.34 68.9325) (end 53.34 78.74) (width 1.5) (layer "B.Cu") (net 23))
 (segment (start 93.98 71.12) (end 109.22 55.88) (width 1.5) (layer "B.Cu") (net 23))
 (segment (start 102.840159 38.1) (end 95.26 30.519841) (width 1.5) (layer "B.Cu") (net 23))
 (segment (start 91.44 83.82) (end 91.44 79.443964) (width 1.5) (layer "B.Cu") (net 23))
 (segment (start 109.22 55.88) (end 109.22 39.37) (width 1.5) (layer "B.Cu") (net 23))
 (segment (start 91.44 79.443964) (end 93.98 76.903964) (width 1.5) (layer "B.Cu") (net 23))
 (segment (start 107.95 38.1) (end 102.840159 38.1) (width 1.5) (layer "B.Cu") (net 23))
 (segment (start 93.98 76.903964) (end 93.98 71.12) (width 1.5) (layer "B.Cu") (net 23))
 (segment (start 109.22 39.37) (end 107.95 38.1) (width 1.5) (layer "B.Cu") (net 23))
 (segment (start 60.96 81.28) (end 58.42 78.74) (width 1.5) (layer "F.Cu") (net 24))
 (segment (start 93.98 81.28) (end 60.96 81.28) (width 1.5) (layer "F.Cu") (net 24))
 (via (at 93.98 81.28) (size 1.5) (drill 0.4) (layers "F.Cu" "B.Cu") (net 24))
 (via (at 58.42 78.74) (size 1.5) (drill 0.4) (layers "F.Cu" "B.Cu") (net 24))
 (segment (start 97.8 29.22) (end 97.8 27.235) (width 1.5) (layer "B.Cu") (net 24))
 (segment (start 109.22 35.56) (end 104.14 35.56) (width 1.5) (layer "B.Cu") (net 24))
 (segment (start 104.14 35.56) (end 97.8 29.22) (width 1.5) (layer "B.Cu") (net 24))
 (segment (start 96.52 73.66) (end 111.76 58.42) (width 1.5) (layer "B.Cu") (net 24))
 (segment (start 111.76 38.1) (end 109.22 35.56) (width 1.5) (layer "B.Cu") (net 24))
 (segment (start 96.52 78.74) (end 96.52 73.66) (width 1.5) (layer "B.Cu") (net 24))
 (segment (start 55.88 68.9325) (end 55.88 76.2) (width 1.5) (layer "B.Cu") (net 24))
 (segment (start 55.88 76.2) (end 58.42 78.74) (width 1.5) (layer "B.Cu") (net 24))
 (segment (start 93.98 81.28) (end 96.52 78.74) (width 1.5) (layer "B.Cu") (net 24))
 (segment (start 111.76 58.42) (end 111.76 38.1) (width 1.5) (layer "B.Cu") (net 24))
 (segment (start 104.14 43.18) (end 101.6 45.72) (width 1.5) (layer "F.Cu") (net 25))
 (segment (start 45.72 50.8) (end 88.9 50.8) (width 1.5) (layer "F.Cu") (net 25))
 (segment (start 45.72 71.12) (end 43.18 68.58) (width 1.5) (layer "F.Cu") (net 25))
 (segment (start 43.18 68.58) (end 43.18 53.34) (width 1.5) (layer "F.Cu") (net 25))
 (segment (start 104.14 30.48) (end 104.14 43.18) (width 1.5) (layer "F.Cu") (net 25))
 (segment (start 43.18 53.34) (end 45.72 50.8) (width 1.5) (layer "F.Cu") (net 25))
 (segment (start 58.42 71.12) (end 45.72 71.12) (width 1.5) (layer "F.Cu") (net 25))
 (segment (start 88.9 50.8) (end 93.98 45.72) (width 1.5) (layer "F.Cu") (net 25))
 (via (at 101.6 45.72) (size 1.5) (drill 0.4) (layers "F.Cu" "B.Cu") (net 25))
 (via (at 58.42 71.12) (size 1.5) (drill 0.4) (layers "F.Cu" "B.Cu") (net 25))
 (via (at 104.14 30.48) (size 1.5) (drill 0.4) (layers "F.Cu" "B.Cu") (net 25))
 (via (at 93.98 45.72) (size 1.5) (drill 0.4) (layers "F.Cu" "B.Cu") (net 25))
 (segment (start 93.98 45.72) (end 101.6 45.72) (width 1.5) (layer "B.Cu") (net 25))
 (segment (start 58.42 68.9325) (end 58.42 71.12) (width 1.5) (layer "B.Cu") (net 25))
 (segment (start 104.14 30.48) (end 100.895 27.235) (width 1.5) (layer "B.Cu") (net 25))
 (segment (start 100.895 27.235) (end 100.34 27.235) (width 1.5) (layer "B.Cu") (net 25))
 (segment (start 60.96 76.2) (end 63.8525 79.0925) (width 1.5) (layer "B.Cu") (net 26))
 (segment (start 60.96 68.9325) (end 60.96 76.2) (width 1.5) (layer "B.Cu") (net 26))
 (segment (start 63.8525 79.0925) (end 67.31 79.0925) (width 1.5) (layer "B.Cu") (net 26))
 (segment (start 66.04 68.9325) (end 66.04 76.2) (width 1.5) (layer "B.Cu") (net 27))
 (segment (start 66.04 76.2) (end 72.39 76.2) (width 1.5) (layer "B.Cu") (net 27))
 (segment (start 72.39 76.2) (end 72.39 79.0925) (width 1.5) (layer "B.Cu") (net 27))
 (segment (start 77.47 77.47) (end 77.47 79.0925) (width 1.5) (layer "B.Cu") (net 28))
 (segment (start 78.74 76.2) (end 77.47 77.47) (width 1.5) (layer "B.Cu") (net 28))
 (segment (start 78.74 68.9325) (end 78.74 76.2) (width 1.5) (layer "B.Cu") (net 28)))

